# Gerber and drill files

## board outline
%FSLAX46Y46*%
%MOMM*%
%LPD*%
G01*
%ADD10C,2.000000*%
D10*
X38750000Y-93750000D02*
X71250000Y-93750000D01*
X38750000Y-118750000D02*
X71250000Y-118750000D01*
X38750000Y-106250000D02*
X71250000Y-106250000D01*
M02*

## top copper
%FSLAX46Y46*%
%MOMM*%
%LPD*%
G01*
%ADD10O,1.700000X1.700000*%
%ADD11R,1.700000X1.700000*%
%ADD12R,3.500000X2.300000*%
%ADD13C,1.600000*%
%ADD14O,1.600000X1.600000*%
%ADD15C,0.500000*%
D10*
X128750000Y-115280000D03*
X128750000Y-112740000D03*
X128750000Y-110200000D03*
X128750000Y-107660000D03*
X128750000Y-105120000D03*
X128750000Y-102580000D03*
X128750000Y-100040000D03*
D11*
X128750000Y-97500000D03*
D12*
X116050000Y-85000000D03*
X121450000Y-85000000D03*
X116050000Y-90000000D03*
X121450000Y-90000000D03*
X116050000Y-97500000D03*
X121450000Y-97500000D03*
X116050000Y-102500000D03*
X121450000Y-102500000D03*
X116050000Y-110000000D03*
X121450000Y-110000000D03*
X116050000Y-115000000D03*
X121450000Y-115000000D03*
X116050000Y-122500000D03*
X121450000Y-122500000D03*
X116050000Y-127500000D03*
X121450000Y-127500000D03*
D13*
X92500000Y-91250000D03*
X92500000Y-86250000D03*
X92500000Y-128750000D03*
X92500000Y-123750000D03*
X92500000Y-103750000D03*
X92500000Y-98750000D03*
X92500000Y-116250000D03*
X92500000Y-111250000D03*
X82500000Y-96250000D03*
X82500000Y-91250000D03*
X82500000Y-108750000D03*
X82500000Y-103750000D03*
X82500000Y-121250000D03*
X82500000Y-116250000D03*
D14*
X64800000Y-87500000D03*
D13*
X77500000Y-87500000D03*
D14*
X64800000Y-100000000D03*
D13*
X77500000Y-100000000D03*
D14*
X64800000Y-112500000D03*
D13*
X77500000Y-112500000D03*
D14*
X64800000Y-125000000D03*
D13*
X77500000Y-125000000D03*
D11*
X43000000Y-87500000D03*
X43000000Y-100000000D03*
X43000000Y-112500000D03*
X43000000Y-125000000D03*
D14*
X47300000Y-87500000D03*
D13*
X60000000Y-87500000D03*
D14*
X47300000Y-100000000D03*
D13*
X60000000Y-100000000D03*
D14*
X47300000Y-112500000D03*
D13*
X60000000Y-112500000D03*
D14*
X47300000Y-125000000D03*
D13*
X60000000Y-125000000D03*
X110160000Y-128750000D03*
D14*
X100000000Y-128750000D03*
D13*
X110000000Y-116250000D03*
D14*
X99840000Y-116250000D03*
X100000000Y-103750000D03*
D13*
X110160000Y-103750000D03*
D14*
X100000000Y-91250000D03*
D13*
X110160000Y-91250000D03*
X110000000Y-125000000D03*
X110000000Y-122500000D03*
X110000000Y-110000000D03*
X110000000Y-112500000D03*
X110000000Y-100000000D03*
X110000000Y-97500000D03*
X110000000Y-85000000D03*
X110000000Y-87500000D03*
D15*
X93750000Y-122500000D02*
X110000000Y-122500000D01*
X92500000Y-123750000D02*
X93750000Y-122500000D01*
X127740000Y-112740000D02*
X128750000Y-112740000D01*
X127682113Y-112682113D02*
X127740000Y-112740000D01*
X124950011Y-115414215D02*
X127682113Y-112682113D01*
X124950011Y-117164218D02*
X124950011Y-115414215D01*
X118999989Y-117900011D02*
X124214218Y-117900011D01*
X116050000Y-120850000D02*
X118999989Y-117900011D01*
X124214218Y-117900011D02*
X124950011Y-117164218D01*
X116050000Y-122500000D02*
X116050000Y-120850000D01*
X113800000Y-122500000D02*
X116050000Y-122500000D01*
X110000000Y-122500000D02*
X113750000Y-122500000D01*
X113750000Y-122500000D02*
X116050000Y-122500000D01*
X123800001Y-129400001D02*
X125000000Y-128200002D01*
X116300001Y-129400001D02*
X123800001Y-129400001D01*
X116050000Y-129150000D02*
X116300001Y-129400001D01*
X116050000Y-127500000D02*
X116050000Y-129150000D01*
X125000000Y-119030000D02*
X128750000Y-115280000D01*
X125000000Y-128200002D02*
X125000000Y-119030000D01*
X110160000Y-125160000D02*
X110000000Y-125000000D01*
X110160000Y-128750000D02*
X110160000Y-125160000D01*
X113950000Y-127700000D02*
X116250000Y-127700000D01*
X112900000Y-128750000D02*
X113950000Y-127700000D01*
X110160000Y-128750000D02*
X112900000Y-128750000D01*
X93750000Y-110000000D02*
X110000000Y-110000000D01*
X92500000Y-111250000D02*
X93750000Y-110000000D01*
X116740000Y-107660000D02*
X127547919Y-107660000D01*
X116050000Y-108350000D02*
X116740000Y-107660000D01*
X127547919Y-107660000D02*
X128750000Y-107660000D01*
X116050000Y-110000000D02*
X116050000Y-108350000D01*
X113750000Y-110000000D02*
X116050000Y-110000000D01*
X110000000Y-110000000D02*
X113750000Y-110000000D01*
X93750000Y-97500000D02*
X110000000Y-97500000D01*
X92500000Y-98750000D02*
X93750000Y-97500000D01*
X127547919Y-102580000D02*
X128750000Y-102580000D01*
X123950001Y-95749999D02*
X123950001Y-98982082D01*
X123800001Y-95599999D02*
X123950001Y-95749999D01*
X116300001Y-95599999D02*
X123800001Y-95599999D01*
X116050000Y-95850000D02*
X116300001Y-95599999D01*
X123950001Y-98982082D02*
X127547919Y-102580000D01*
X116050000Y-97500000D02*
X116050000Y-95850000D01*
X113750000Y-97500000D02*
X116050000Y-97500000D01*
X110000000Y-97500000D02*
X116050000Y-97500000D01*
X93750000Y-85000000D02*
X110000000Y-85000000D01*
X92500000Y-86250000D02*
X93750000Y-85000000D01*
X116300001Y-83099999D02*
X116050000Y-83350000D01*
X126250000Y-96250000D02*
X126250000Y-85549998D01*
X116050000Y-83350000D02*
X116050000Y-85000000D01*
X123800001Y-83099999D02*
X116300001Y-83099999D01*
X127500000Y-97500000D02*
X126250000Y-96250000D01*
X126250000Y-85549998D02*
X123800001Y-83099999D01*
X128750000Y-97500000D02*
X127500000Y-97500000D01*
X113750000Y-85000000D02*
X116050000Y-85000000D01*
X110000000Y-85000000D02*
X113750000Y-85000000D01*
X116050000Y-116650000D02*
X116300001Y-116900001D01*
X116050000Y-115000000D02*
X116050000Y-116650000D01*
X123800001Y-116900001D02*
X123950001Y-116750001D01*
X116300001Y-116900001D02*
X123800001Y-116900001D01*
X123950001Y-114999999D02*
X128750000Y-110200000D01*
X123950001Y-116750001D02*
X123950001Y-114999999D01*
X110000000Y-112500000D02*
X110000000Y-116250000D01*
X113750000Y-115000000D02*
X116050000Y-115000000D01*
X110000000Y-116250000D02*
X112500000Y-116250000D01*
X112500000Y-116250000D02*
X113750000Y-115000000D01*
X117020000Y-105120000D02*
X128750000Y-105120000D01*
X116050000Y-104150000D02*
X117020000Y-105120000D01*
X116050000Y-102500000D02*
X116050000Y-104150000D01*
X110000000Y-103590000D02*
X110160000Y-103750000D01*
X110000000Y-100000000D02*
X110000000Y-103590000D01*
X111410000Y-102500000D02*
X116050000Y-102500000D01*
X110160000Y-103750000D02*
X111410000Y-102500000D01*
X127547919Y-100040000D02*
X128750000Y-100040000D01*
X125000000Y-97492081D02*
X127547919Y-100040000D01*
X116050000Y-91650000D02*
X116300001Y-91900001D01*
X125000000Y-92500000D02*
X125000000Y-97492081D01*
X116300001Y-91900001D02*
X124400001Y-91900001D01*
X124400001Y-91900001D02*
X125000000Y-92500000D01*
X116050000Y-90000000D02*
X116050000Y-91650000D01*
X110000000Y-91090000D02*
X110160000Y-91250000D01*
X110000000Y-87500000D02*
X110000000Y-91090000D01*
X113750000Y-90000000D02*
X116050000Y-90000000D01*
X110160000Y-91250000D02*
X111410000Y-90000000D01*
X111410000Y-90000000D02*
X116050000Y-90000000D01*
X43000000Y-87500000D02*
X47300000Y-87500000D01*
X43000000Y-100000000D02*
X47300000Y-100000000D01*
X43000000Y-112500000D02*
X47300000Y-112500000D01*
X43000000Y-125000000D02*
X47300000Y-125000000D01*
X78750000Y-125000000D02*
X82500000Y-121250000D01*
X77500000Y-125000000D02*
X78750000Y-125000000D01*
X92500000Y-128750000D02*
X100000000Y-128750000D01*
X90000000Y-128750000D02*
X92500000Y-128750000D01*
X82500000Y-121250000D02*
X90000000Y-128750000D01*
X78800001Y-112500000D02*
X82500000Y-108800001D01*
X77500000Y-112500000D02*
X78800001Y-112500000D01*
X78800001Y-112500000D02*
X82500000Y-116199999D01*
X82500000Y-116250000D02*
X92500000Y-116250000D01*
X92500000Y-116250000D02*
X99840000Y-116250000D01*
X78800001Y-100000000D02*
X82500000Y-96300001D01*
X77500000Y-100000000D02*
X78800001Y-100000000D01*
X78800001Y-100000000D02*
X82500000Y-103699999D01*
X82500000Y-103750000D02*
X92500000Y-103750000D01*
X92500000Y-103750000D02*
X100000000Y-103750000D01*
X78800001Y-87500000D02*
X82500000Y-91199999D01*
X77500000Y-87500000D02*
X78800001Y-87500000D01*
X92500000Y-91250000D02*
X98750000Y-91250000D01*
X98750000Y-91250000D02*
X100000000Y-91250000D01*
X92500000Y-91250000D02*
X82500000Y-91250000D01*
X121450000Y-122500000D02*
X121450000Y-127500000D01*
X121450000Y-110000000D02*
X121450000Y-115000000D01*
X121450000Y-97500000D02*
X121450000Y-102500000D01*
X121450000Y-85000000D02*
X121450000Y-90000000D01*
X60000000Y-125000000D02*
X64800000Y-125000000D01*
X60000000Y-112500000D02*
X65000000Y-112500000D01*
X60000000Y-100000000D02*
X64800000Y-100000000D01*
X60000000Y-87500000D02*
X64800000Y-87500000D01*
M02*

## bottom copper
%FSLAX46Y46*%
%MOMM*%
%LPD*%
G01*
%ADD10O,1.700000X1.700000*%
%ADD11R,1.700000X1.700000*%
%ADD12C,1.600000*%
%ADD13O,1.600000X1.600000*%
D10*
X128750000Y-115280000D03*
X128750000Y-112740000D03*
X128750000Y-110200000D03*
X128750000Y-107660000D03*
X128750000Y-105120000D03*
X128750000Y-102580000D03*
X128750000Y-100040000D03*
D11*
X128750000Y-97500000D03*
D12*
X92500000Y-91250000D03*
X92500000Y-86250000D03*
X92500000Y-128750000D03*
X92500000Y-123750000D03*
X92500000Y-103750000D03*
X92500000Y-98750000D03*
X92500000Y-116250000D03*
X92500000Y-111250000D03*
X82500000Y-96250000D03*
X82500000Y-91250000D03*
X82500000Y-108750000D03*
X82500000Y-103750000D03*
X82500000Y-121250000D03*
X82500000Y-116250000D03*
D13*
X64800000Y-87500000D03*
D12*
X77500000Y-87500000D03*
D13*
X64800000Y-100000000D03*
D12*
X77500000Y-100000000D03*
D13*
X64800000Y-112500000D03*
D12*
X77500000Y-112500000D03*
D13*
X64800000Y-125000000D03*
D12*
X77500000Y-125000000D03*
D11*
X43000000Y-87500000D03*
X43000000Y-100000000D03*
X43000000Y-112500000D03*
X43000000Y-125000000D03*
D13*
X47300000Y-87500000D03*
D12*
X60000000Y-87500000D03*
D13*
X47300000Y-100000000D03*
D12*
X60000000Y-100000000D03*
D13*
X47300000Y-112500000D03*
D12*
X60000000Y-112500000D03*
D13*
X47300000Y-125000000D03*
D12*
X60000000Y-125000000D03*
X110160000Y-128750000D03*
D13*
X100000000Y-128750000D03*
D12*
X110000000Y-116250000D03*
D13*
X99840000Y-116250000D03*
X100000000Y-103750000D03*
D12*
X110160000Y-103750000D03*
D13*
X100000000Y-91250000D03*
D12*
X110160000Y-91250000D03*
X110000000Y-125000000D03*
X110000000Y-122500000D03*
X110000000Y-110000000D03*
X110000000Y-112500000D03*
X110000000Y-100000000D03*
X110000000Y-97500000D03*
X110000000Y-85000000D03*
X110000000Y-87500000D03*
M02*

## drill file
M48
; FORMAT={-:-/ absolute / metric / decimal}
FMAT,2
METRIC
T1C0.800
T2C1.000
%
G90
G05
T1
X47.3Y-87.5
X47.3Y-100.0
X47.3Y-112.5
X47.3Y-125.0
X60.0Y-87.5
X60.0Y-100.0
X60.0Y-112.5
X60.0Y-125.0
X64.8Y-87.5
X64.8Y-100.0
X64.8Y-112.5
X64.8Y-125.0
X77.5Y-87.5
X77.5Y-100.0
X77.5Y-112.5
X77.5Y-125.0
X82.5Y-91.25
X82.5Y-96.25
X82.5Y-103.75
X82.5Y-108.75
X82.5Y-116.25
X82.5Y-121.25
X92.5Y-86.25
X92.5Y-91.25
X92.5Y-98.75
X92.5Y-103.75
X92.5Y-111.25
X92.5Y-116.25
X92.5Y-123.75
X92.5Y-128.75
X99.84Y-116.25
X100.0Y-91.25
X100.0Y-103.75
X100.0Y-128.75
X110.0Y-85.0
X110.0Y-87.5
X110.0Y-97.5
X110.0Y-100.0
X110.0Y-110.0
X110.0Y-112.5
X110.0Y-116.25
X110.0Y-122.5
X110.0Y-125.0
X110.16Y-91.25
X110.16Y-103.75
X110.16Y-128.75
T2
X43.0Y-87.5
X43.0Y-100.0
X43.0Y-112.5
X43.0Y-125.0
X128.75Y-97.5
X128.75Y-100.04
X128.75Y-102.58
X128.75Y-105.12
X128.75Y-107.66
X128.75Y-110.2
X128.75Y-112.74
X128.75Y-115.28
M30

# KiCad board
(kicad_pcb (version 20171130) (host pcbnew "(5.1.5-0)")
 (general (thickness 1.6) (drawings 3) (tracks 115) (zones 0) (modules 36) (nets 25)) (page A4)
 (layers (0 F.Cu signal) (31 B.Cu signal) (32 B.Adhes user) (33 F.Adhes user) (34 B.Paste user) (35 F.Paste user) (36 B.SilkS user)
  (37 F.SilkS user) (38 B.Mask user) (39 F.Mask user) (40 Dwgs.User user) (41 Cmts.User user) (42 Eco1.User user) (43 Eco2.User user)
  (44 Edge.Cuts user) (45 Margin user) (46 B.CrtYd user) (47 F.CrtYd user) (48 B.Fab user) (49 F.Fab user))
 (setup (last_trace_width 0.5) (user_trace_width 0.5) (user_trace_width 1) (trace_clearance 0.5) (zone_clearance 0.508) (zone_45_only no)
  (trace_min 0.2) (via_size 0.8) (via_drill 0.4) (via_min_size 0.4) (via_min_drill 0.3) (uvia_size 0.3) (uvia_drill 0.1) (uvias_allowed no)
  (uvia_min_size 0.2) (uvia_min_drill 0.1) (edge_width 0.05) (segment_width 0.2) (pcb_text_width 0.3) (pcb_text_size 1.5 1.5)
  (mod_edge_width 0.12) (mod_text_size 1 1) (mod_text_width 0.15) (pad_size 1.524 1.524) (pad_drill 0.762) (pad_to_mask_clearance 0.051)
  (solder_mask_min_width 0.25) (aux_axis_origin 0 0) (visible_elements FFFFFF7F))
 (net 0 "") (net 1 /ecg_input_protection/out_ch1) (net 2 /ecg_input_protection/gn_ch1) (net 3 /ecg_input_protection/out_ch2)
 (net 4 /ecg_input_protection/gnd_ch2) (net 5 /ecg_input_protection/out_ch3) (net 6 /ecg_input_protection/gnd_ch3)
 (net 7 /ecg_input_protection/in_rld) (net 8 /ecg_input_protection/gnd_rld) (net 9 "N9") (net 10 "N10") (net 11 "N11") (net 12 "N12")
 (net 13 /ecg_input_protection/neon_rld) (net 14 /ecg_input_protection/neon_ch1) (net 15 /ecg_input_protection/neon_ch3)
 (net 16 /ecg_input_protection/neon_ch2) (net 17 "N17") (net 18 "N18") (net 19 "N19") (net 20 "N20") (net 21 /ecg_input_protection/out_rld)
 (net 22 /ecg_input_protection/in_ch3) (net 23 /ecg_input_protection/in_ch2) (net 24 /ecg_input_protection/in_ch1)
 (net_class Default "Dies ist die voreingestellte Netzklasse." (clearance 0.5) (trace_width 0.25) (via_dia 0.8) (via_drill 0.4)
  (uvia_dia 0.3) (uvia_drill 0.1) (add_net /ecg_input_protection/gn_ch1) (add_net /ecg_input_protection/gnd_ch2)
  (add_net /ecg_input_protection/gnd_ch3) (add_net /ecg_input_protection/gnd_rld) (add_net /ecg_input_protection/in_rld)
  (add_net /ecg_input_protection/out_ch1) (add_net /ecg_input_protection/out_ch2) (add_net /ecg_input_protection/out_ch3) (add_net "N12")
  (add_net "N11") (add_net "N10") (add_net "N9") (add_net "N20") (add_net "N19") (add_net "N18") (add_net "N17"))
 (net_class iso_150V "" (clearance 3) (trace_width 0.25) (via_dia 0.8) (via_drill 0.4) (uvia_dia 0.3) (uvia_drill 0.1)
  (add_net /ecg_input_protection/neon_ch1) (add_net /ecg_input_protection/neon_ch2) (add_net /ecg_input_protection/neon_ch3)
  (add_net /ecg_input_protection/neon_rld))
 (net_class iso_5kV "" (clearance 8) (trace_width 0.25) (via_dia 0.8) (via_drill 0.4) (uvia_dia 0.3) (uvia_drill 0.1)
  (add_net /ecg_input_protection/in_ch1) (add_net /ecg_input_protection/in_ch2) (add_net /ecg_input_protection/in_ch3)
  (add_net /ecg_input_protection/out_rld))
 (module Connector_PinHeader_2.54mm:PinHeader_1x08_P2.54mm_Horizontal (layer F.Cu) (at 128.75 97.5)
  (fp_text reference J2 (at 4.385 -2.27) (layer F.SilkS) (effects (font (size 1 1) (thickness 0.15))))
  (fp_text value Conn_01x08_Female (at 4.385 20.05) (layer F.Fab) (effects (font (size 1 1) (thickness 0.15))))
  (pad 8 thru_hole oval (at 0 17.78) (size 1.7 1.7) (drill 1) (layers *.Cu *.Mask) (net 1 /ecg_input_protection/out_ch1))
  (pad 7 thru_hole oval (at 0 15.24) (size 1.7 1.7) (drill 1) (layers *.Cu *.Mask) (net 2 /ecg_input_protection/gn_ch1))
  (pad 6 thru_hole oval (at 0 12.7) (size 1.7 1.7) (drill 1) (layers *.Cu *.Mask) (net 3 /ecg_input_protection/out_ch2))
  (pad 5 thru_hole oval (at 0 10.16) (size 1.7 1.7) (drill 1) (layers *.Cu *.Mask) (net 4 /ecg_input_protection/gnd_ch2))
  (pad 4 thru_hole oval (at 0 7.62) (size 1.7 1.7) (drill 1) (layers *.Cu *.Mask) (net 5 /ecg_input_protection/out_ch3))
  (pad 3 thru_hole oval (at 0 5.08) (size 1.7 1.7) (drill 1) (layers *.Cu *.Mask) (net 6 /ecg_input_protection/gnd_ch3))
  (pad 2 thru_hole oval (at 0 2.54) (size 1.7 1.7) (drill 1) (layers *.Cu *.Mask) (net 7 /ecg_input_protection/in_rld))
  (pad 1 thru_hole rect (at 0 0) (size 1.7 1.7) (drill 1) (layers *.Cu *.Mask) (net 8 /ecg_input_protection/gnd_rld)))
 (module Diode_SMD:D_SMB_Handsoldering (layer F.Cu) (at 118.75 85 180)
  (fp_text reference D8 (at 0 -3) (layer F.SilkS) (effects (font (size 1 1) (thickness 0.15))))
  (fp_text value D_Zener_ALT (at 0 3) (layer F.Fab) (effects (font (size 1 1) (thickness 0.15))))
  (pad 2 smd rect (at 2.7 0 180) (size 3.5 2.3) (layers F.Cu F.Paste F.Mask) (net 8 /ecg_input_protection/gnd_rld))
  (pad 1 smd rect (at -2.7 0 180) (size 3.5 2.3) (layers F.Cu F.Paste F.Mask) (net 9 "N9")))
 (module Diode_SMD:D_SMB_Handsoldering (layer F.Cu) (at 118.75 90 180)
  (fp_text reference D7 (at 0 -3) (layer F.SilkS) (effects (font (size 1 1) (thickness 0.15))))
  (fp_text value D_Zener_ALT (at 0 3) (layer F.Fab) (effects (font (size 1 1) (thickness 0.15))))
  (pad 2 smd rect (at 2.7 0 180) (size 3.5 2.3) (layers F.Cu F.Paste F.Mask) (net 7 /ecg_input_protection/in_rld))
  (pad 1 smd rect (at -2.7 0 180) (size 3.5 2.3) (layers F.Cu F.Paste F.Mask) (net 9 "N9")))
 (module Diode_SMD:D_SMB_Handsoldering (layer F.Cu) (at 118.75 97.5 180)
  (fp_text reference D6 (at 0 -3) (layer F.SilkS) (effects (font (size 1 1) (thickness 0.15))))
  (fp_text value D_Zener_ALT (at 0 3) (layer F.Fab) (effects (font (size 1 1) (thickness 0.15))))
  (pad 2 smd rect (at 2.7 0 180) (size 3.5 2.3) (layers F.Cu F.Paste F.Mask) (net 6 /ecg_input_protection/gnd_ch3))
  (pad 1 smd rect (at -2.7 0 180) (size 3.5 2.3) (layers F.Cu F.Paste F.Mask) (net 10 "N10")))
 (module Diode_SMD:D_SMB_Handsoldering (layer F.Cu) (at 118.75 102.5 180)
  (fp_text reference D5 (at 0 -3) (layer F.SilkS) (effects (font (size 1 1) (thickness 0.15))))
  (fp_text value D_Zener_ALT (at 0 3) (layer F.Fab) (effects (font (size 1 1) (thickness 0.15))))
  (pad 2 smd rect (at 2.7 0 180) (size 3.5 2.3) (layers F.Cu F.Paste F.Mask) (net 5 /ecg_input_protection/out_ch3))
  (pad 1 smd rect (at -2.7 0 180) (size 3.5 2.3) (layers F.Cu F.Paste F.Mask) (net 10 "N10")))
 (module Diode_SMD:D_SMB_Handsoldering (layer F.Cu) (at 118.75 110 180)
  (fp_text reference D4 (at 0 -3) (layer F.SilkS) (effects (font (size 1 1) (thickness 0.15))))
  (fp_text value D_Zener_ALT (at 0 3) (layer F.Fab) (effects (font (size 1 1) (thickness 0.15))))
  (pad 2 smd rect (at 2.7 0 180) (size 3.5 2.3) (layers F.Cu F.Paste F.Mask) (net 4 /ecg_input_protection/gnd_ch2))
  (pad 1 smd rect (at -2.7 0 180) (size 3.5 2.3) (layers F.Cu F.Paste F.Mask) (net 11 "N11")))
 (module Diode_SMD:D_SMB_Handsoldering (layer F.Cu) (at 118.75 115 180)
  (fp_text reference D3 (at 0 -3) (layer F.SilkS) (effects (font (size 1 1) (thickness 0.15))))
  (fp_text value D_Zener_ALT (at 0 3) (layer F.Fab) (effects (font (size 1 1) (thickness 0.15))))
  (pad 2 smd rect (at 2.7 0 180) (size 3.5 2.3) (layers F.Cu F.Paste F.Mask) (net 3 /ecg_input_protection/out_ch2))
  (pad 1 smd rect (at -2.7 0 180) (size 3.5 2.3) (layers F.Cu F.Paste F.Mask) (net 11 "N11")))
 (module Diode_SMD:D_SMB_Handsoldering (layer F.Cu) (at 118.75 122.5 180)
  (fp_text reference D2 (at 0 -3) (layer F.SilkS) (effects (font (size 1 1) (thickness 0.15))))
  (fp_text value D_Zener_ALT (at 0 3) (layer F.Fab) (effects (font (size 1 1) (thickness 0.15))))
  (pad 2 smd rect (at 2.7 0 180) (size 3.5 2.3) (layers F.Cu F.Paste F.Mask) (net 2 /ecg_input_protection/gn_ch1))
  (pad 1 smd rect (at -2.7 0 180) (size 3.5 2.3) (layers F.Cu F.Paste F.Mask) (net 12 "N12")))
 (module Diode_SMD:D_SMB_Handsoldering (layer F.Cu) (at 118.75 127.5 180)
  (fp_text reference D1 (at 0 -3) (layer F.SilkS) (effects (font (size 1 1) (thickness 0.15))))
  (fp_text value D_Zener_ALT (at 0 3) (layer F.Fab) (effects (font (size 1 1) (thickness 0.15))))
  (pad 2 smd rect (at 2.7 0 180) (size 3.5 2.3) (layers F.Cu F.Paste F.Mask) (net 1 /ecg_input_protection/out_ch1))
  (pad 1 smd rect (at -2.7 0 180) (size 3.5 2.3) (layers F.Cu F.Paste F.Mask) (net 12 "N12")))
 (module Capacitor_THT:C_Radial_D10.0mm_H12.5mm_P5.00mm (layer F.Cu) (at 92.5 86.25 270)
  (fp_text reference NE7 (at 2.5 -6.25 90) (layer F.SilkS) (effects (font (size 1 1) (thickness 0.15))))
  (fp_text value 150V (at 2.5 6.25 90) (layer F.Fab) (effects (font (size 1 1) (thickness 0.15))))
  (pad 2 thru_hole circle (at 5 0 270) (size 1.6 1.6) (drill 0.8) (layers *.Cu *.Mask) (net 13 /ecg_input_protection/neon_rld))
  (pad 1 thru_hole circle (at 0 0 270) (size 1.6 1.6) (drill 0.8) (layers *.Cu *.Mask) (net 8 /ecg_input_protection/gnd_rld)))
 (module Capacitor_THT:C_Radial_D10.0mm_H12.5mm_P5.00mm (layer F.Cu) (at 92.5 123.75 270)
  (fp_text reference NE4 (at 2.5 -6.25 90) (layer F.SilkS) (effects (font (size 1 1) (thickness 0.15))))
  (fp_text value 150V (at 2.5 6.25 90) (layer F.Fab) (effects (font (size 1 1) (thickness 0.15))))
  (pad 2 thru_hole circle (at 5 0 270) (size 1.6 1.6) (drill 0.8) (layers *.Cu *.Mask) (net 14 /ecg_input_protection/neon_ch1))
  (pad 1 thru_hole circle (at 0 0 270) (size 1.6 1.6) (drill 0.8) (layers *.Cu *.Mask) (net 2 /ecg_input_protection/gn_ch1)))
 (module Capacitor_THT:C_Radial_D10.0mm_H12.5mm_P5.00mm (layer F.Cu) (at 92.5 98.75 270)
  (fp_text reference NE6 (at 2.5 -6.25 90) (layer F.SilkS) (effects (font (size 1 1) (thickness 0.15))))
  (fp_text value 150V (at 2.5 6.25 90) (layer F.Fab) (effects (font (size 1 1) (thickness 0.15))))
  (pad 2 thru_hole circle (at 5 0 270) (size 1.6 1.6) (drill 0.8) (layers *.Cu *.Mask) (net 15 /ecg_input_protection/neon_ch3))
  (pad 1 thru_hole circle (at 0 0 270) (size 1.6 1.6) (drill 0.8) (layers *.Cu *.Mask) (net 6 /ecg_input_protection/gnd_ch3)))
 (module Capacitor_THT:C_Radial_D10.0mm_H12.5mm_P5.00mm (layer F.Cu) (at 92.5 111.25 270)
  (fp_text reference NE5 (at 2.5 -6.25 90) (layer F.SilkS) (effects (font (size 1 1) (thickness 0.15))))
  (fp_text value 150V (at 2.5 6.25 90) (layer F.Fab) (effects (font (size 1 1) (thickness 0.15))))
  (pad 2 thru_hole circle (at 5 0 270) (size 1.6 1.6) (drill 0.8) (layers *.Cu *.Mask) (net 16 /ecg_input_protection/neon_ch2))
  (pad 1 thru_hole circle (at 0 0 270) (size 1.6 1.6) (drill 0.8) (layers *.Cu *.Mask) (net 4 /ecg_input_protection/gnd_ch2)))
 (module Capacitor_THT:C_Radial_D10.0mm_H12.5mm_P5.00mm (layer F.Cu) (at 82.5 91.25 270)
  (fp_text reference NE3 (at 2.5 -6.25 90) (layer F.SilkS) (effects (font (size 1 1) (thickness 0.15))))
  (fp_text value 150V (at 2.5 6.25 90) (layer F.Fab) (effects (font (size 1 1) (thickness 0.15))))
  (pad 2 thru_hole circle (at 5 0 270) (size 1.6 1.6) (drill 0.8) (layers *.Cu *.Mask) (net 15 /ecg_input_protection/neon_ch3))
  (pad 1 thru_hole circle (at 0 0 270) (size 1.6 1.6) (drill 0.8) (layers *.Cu *.Mask) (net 13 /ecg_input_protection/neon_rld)))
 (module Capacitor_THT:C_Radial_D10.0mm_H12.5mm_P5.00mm (layer F.Cu) (at 82.5 103.75 270)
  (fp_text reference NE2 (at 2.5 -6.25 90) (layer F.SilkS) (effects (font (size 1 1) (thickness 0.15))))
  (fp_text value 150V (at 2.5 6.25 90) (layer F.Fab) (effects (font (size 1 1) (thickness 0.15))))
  (pad 2 thru_hole circle (at 5 0 270) (size 1.6 1.6) (drill 0.8) (layers *.Cu *.Mask) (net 16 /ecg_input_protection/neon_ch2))
  (pad 1 thru_hole circle (at 0 0 270) (size 1.6 1.6) (drill 0.8) (layers *.Cu *.Mask) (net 15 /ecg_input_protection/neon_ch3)))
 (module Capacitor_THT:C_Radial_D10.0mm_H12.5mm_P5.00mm (layer F.Cu) (at 82.5 116.25 270)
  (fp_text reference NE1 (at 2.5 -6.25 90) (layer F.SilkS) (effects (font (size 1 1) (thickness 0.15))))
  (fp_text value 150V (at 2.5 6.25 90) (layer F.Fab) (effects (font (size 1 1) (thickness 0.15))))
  (pad 2 thru_hole circle (at 5 0 270) (size 1.6 1.6) (drill 0.8) (layers *.Cu *.Mask) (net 14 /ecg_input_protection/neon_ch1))
  (pad 1 thru_hole circle (at 0 0 270) (size 1.6 1.6) (drill 0.8) (layers *.Cu *.Mask) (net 16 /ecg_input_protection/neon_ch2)))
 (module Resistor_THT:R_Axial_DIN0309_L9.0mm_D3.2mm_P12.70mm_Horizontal (layer F.Cu) (at 77.5 87.5 180)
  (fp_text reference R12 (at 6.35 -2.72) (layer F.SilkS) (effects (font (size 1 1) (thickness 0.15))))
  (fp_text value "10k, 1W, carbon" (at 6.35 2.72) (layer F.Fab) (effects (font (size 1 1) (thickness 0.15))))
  (pad 2 thru_hole oval (at 12.7 0 180) (size 1.6 1.6) (drill 0.8) (layers *.Cu *.Mask) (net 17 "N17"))
  (pad 1 thru_hole circle (at 0 0 180) (size 1.6 1.6) (drill 0.8) (layers *.Cu *.Mask) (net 13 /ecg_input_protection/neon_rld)))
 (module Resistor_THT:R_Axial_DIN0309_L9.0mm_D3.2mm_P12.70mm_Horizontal (layer F.Cu) (at 77.5 100 180)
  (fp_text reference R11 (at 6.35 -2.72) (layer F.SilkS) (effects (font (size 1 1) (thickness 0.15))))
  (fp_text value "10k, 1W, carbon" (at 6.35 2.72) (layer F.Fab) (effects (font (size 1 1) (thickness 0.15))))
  (pad 2 thru_hole oval (at 12.7 0 180) (size 1.6 1.6) (drill 0.8) (layers *.Cu *.Mask) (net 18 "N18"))
  (pad 1 thru_hole circle (at 0 0 180) (size 1.6 1.6) (drill 0.8) (layers *.Cu *.Mask) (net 15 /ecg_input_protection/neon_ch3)))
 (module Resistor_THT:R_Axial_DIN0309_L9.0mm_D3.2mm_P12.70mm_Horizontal (layer F.Cu) (at 77.5 112.5 180)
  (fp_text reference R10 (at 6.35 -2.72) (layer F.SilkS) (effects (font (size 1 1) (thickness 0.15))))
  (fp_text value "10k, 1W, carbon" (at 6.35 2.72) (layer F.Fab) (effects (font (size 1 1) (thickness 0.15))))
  (pad 2 thru_hole oval (at 12.7 0 180) (size 1.6 1.6) (drill 0.8) (layers *.Cu *.Mask) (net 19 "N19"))
  (pad 1 thru_hole circle (at 0 0 180) (size 1.6 1.6) (drill 0.8) (layers *.Cu *.Mask) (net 16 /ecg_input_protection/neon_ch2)))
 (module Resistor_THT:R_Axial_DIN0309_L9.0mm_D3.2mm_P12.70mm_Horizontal (layer F.Cu) (at 77.5 125 180)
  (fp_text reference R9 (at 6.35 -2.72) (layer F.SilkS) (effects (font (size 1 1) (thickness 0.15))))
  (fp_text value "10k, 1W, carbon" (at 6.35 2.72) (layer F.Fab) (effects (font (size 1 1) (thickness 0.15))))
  (pad 2 thru_hole oval (at 12.7 0 180) (size 1.6 1.6) (drill 0.8) (layers *.Cu *.Mask) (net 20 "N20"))
  (pad 1 thru_hole circle (at 0 0 180) (size 1.6 1.6) (drill 0.8) (layers *.Cu *.Mask) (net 14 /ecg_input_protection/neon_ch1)))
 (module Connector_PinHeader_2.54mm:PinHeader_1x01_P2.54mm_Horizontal (layer F.Cu) (at 43 87.5 180)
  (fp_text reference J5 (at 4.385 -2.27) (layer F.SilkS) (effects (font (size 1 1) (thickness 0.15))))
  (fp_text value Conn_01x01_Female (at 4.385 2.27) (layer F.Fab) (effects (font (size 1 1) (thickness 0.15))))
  (pad 1 thru_hole rect (at 0 0 180) (size 1.7 1.7) (drill 1) (layers *.Cu *.Mask) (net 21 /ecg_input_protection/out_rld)))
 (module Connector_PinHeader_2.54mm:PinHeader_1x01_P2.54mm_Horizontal (layer F.Cu) (at 43 100 180)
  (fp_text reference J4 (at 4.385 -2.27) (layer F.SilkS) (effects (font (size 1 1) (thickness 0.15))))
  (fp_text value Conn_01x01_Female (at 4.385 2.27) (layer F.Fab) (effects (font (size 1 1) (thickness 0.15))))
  (pad 1 thru_hole rect (at 0 0 180) (size 1.7 1.7) (drill 1) (layers *.Cu *.Mask) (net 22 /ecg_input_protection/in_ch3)))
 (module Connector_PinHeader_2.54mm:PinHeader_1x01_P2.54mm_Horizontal (layer F.Cu) (at 43 112.5 180)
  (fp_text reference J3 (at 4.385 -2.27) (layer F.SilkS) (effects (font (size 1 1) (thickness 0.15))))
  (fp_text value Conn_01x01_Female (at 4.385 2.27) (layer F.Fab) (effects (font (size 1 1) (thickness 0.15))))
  (pad 1 thru_hole rect (at 0 0 180) (size 1.7 1.7) (drill 1) (layers *.Cu *.Mask) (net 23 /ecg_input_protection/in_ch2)))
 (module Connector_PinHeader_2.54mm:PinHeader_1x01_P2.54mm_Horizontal (layer F.Cu) (at 43 125 180)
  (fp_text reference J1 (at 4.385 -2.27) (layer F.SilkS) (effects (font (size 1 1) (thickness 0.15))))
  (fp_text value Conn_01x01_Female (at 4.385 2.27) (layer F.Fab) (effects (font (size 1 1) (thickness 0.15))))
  (pad 1 thru_hole rect (at 0 0 180) (size 1.7 1.7) (drill 1) (layers *.Cu *.Mask) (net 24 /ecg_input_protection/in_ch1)))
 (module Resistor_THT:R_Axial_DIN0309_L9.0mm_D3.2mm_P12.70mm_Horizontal (layer F.Cu) (at 60 87.5 180)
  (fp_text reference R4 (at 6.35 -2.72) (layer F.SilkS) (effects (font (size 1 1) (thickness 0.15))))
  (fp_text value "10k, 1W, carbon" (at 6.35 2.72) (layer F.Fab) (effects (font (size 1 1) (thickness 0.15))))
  (pad 2 thru_hole oval (at 12.7 0 180) (size 1.6 1.6) (drill 0.8) (layers *.Cu *.Mask) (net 21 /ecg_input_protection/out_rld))
  (pad 1 thru_hole circle (at 0 0 180) (size 1.6 1.6) (drill 0.8) (layers *.Cu *.Mask) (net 17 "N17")))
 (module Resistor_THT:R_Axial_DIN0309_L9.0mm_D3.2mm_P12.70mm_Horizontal (layer F.Cu) (at 60 100 180)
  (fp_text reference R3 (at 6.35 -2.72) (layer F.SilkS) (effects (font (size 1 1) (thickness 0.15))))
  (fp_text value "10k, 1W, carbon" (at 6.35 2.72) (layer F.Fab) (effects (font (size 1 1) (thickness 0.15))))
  (pad 2 thru_hole oval (at 12.7 0 180) (size 1.6 1.6) (drill 0.8) (layers *.Cu *.Mask) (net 22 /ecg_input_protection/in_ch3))
  (pad 1 thru_hole circle (at 0 0 180) (size 1.6 1.6) (drill 0.8) (layers *.Cu *.Mask) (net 18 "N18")))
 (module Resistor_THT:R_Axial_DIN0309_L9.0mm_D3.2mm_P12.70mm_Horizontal (layer F.Cu) (at 60 112.5 180)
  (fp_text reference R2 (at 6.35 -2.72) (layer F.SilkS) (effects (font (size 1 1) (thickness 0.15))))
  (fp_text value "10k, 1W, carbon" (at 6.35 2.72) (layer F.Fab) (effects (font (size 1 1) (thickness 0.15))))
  (pad 2 thru_hole oval (at 12.7 0 180) (size 1.6 1.6) (drill 0.8) (layers *.Cu *.Mask) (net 23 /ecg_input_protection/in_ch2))
  (pad 1 thru_hole circle (at 0 0 180) (size 1.6 1.6) (drill 0.8) (layers *.Cu *.Mask) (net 19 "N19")))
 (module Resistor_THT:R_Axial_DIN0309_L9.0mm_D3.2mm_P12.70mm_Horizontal (layer F.Cu) (at 60 125 180)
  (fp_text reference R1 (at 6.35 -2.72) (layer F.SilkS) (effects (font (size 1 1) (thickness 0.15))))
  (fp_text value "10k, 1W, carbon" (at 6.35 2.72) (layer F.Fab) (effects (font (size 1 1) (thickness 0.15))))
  (pad 2 thru_hole oval (at 12.7 0 180) (size 1.6 1.6) (drill 0.8) (layers *.Cu *.Mask) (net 24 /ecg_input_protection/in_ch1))
  (pad 1 thru_hole circle (at 0 0 180) (size 1.6 1.6) (drill 0.8) (layers *.Cu *.Mask) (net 20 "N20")))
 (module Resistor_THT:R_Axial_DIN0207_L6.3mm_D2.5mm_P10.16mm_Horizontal (layer F.Cu) (at 110.16 128.75 180)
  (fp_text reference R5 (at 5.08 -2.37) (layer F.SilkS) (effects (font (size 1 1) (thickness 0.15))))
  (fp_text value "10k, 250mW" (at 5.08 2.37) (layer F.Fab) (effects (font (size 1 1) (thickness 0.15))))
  (pad 1 thru_hole circle (at 0 0 180) (size 1.6 1.6) (drill 0.8) (layers *.Cu *.Mask) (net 1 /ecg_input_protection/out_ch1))
  (pad 2 thru_hole oval (at 10.16 0 180) (size 1.6 1.6) (drill 0.8) (layers *.Cu *.Mask) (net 14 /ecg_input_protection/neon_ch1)))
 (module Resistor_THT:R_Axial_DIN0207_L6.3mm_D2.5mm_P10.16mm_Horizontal (layer F.Cu) (at 110 116.25 180)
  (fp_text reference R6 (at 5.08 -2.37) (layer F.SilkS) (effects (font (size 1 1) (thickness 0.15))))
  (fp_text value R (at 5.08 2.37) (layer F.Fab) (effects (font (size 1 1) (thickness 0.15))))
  (pad 1 thru_hole circle (at 0 0 180) (size 1.6 1.6) (drill 0.8) (layers *.Cu *.Mask) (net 3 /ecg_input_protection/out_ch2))
  (pad 2 thru_hole oval (at 10.16 0 180) (size 1.6 1.6) (drill 0.8) (layers *.Cu *.Mask) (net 16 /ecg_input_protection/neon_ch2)))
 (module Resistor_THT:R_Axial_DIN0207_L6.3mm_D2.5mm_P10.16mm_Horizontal (layer F.Cu) (at 110.16 103.75 180)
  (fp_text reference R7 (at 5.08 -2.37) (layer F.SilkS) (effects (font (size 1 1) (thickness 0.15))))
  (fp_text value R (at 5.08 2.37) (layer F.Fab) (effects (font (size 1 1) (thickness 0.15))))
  (pad 2 thru_hole oval (at 10.16 0 180) (size 1.6 1.6) (drill 0.8) (layers *.Cu *.Mask) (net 15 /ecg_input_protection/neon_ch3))
  (pad 1 thru_hole circle (at 0 0 180) (size 1.6 1.6) (drill 0.8) (layers *.Cu *.Mask) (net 5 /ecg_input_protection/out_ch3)))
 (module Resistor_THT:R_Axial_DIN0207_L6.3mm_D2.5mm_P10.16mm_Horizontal (layer F.Cu) (at 110.16 91.25 180)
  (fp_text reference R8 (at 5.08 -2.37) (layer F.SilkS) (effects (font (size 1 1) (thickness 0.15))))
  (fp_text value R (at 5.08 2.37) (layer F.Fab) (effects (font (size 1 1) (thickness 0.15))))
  (pad 2 thru_hole oval (at 10.16 0 180) (size 1.6 1.6) (drill 0.8) (layers *.Cu *.Mask) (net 13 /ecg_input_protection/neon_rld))
  (pad 1 thru_hole circle (at 0 0 180) (size 1.6 1.6) (drill 0.8) (layers *.Cu *.Mask) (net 7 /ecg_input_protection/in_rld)))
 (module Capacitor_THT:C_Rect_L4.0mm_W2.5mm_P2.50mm (layer F.Cu) (at 110 125 90)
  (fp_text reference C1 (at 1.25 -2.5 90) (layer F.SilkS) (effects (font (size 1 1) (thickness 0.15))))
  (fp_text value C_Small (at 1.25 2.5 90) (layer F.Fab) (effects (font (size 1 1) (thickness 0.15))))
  (pad 1 thru_hole circle (at 0 0 90) (size 1.6 1.6) (drill 0.8) (layers *.Cu *.Mask) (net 1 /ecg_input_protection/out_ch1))
  (pad 2 thru_hole circle (at 2.5 0 90) (size 1.6 1.6) (drill 0.8) (layers *.Cu *.Mask) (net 2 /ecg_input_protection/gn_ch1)))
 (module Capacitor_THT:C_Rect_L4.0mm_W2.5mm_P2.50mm (layer F.Cu) (at 110 112.5 90)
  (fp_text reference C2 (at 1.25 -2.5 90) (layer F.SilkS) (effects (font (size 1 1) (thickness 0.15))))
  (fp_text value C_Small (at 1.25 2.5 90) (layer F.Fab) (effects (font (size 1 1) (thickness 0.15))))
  (pad 2 thru_hole circle (at 2.5 0 90) (size 1.6 1.6) (drill 0.8) (layers *.Cu *.Mask) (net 4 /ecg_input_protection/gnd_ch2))
  (pad 1 thru_hole circle (at 0 0 90) (size 1.6 1.6) (drill 0.8) (layers *.Cu *.Mask) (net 3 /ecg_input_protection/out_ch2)))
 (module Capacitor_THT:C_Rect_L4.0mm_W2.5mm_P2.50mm (layer F.Cu) (at 110 100 90)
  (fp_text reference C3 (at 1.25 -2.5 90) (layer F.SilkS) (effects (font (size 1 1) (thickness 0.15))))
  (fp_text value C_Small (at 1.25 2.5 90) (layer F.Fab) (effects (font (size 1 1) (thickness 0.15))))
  (pad 1 thru_hole circle (at 0 0 90) (size 1.6 1.6) (drill 0.8) (layers *.Cu *.Mask) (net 5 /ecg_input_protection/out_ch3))
  (pad 2 thru_hole circle (at 2.5 0 90) (size 1.6 1.6) (drill 0.8) (layers *.Cu *.Mask) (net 6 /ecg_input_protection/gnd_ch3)))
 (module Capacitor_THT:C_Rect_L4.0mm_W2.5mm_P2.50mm (layer F.Cu) (at 110 87.5 90)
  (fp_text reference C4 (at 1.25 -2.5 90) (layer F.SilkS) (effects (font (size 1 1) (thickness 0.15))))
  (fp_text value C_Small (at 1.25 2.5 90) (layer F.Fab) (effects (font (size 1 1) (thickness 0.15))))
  (pad 2 thru_hole circle (at 2.5 0 90) (size 1.6 1.6) (drill 0.8) (layers *.Cu *.Mask) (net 8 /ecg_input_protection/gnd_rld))
  (pad 1 thru_hole circle (at 0 0 90) (size 1.6 1.6) (drill 0.8) (layers *.Cu *.Mask) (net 7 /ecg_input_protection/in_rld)))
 (gr_line (start 38.75 93.75) (end 71.25 93.75) (layer Edge.Cuts) (width 2))
 (gr_line (start 38.75 118.75) (end 71.25 118.75) (layer Edge.Cuts) (width 2))
 (gr_line (start 38.75 106.25) (end 71.25 106.25) (layer Edge.Cuts) (width 2))
 (segment (start 93.75 122.5) (end 110 122.5) (width 0.5) (layer F.Cu) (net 2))
 (segment (start 92.5 123.75) (end 93.75 122.5) (width 0.5) (layer F.Cu) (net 2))
 (segment (start 127.74 112.74) (end 128.75 112.74) (width 0.5) (layer F.Cu) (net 2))
 (segment (start 127.682113 112.682113) (end 127.74 112.74) (width 0.5) (layer F.Cu) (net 2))
 (segment (start 124.950011 115.414215) (end 127.682113 112.682113) (width 0.5) (layer F.Cu) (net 2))
 (segment (start 124.950011 117.164218) (end 124.950011 115.414215) (width 0.5) (layer F.Cu) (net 2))
 (segment (start 118.999989 117.900011) (end 124.214218 117.900011) (width 0.5) (layer F.Cu) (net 2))
 (segment (start 116.05 120.85) (end 118.999989 117.900011) (width 0.5) (layer F.Cu) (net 2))
 (segment (start 124.214218 117.900011) (end 124.950011 117.164218) (width 0.5) (layer F.Cu) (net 2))
 (segment (start 116.05 122.5) (end 116.05 120.85) (width 0.5) (layer F.Cu) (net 2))
 (segment (start 113.8 122.5) (end 116.05 122.5) (width 0.5) (layer F.Cu) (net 2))
 (segment (start 110 122.5) (end 113.75 122.5) (width 0.5) (layer F.Cu) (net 2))
 (segment (start 113.75 122.5) (end 116.05 122.5) (width 0.5) (layer F.Cu) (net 2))
 (segment (start 123.800001 129.400001) (end 125 128.200002) (width 0.5) (layer F.Cu) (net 1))
 (segment (start 116.300001 129.400001) (end 123.800001 129.400001) (width 0.5) (layer F.Cu) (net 1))
 (segment (start 116.05 129.15) (end 116.300001 129.400001) (width 0.5) (layer F.Cu) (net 1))
 (segment (start 116.05 127.5) (end 116.05 129.15) (width 0.5) (layer F.Cu) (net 1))
 (segment (start 125 119.03) (end 128.75 115.28) (width 0.5) (layer F.Cu) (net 1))
 (segment (start 125 128.200002) (end 125 119.03) (width 0.5) (layer F.Cu) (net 1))
 (segment (start 110.16 125.16) (end 110 125) (width 0.5) (layer F.Cu) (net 1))
 (segment (start 110.16 128.75) (end 110.16 125.16) (width 0.5) (layer F.Cu) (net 1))
 (segment (start 113.95 127.7) (end 116.25 127.7) (width 0.5) (layer F.Cu) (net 1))
 (segment (start 112.9 128.75) (end 113.95 127.7) (width 0.5) (layer F.Cu) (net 1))
 (segment (start 110.16 128.75) (end 112.9 128.75) (width 0.5) (layer F.Cu) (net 1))
 (segment (start 93.75 110) (end 110 110) (width 0.5) (layer F.Cu) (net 4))
 (segment (start 92.5 111.25) (end 93.75 110) (width 0.5) (layer F.Cu) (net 4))
 (segment (start 116.74 107.66) (end 127.547919 107.66) (width 0.5) (layer F.Cu) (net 4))
 (segment (start 116.05 108.35) (end 116.74 107.66) (width 0.5) (layer F.Cu) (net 4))
 (segment (start 127.547919 107.66) (end 128.75 107.66) (width 0.5) (layer F.Cu) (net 4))
 (segment (start 116.05 110) (end 116.05 108.35) (width 0.5) (layer F.Cu) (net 4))
 (segment (start 113.75 110) (end 116.05 110) (width 0.5) (layer F.Cu) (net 4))
 (segment (start 110 110) (end 113.75 110) (width 0.5) (layer F.Cu) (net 4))
 (segment (start 93.75 97.5) (end 110 97.5) (width 0.5) (layer F.Cu) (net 6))
 (segment (start 92.5 98.75) (end 93.75 97.5) (width 0.5) (layer F.Cu) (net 6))
 (segment (start 127.547919 102.58) (end 128.75 102.58) (width 0.5) (layer F.Cu) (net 6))
 (segment (start 123.950001 95.749999) (end 123.950001 98.982082) (width 0.5) (layer F.Cu) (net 6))
 (segment (start 123.800001 95.599999) (end 123.950001 95.749999) (width 0.5) (layer F.Cu) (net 6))
 (segment (start 116.300001 95.599999) (end 123.800001 95.599999) (width 0.5) (layer F.Cu) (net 6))
 (segment (start 116.05 95.85) (end 116.300001 95.599999) (width 0.5) (layer F.Cu) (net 6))
 (segment (start 123.950001 98.982082) (end 127.547919 102.58) (width 0.5) (layer F.Cu) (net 6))
 (segment (start 116.05 97.5) (end 116.05 95.85) (width 0.5) (layer F.Cu) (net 6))
 (segment (start 113.75 97.5) (end 116.05 97.5) (width 0.5) (layer F.Cu) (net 6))
 (segment (start 110 97.5) (end 116.05 97.5) (width 0.5) (layer F.Cu) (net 6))
 (segment (start 93.75 85) (end 110 85) (width 0.5) (layer F.Cu) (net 8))
 (segment (start 92.5 86.25) (end 93.75 85) (width 0.5) (layer F.Cu) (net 8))
 (segment (start 116.300001 83.099999) (end 116.05 83.35) (width 0.5) (layer F.Cu) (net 8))
 (segment (start 126.25 96.25) (end 126.25 85.549998) (width 0.5) (layer F.Cu) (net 8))
 (segment (start 116.05 83.35) (end 116.05 85) (width 0.5) (layer F.Cu) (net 8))
 (segment (start 123.800001 83.099999) (end 116.300001 83.099999) (width 0.5) (layer F.Cu) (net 8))
 (segment (start 127.5 97.5) (end 126.25 96.25) (width 0.5) (layer F.Cu) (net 8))
 (segment (start 126.25 85.549998) (end 123.800001 83.099999) (width 0.5) (layer F.Cu) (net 8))
 (segment (start 128.75 97.5) (end 127.5 97.5) (width 0.5) (layer F.Cu) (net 8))
 (segment (start 113.75 85) (end 116.05 85) (width 0.5) (layer F.Cu) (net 8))
 (segment (start 110 85) (end 113.75 85) (width 0.5) (layer F.Cu) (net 8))
 (segment (start 116.05 116.65) (end 116.300001 116.900001) (width 0.5) (layer F.Cu) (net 3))
 (segment (start 116.05 115) (end 116.05 116.65) (width 0.5) (layer F.Cu) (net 3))
 (segment (start 123.800001 116.900001) (end 123.950001 116.750001) (width 0.5) (layer F.Cu) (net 3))
 (segment (start 116.300001 116.900001) (end 123.800001 116.900001) (width 0.5) (layer F.Cu) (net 3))
 (segment (start 123.950001 114.999999) (end 128.75 110.2) (width 0.5) (layer F.Cu) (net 3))
 (segment (start 123.950001 116.750001) (end 123.950001 114.999999) (width 0.5) (layer F.Cu) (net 3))
 (segment (start 110 112.5) (end 110 116.25) (width 0.5) (layer F.Cu) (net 3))
 (segment (start 113.75 115) (end 116.05 115) (width 0.5) (layer F.Cu) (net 3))
 (segment (start 110 116.25) (end 112.5 116.25) (width 0.5) (layer F.Cu) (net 3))
 (segment (start 112.5 116.25) (end 113.75 115) (width 0.5) (layer F.Cu) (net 3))
 (segment (start 117.02 105.12) (end 128.75 105.12) (width 0.5) (layer F.Cu) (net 5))
 (segment (start 116.05 104.15) (end 117.02 105.12) (width 0.5) (layer F.Cu) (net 5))
 (segment (start 116.05 102.5) (end 116.05 104.15) (width 0.5) (layer F.Cu) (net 5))
 (segment (start 110 103.59) (end 110.16 103.75) (width 0.5) (layer F.Cu) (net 5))
 (segment (start 110 100) (end 110 103.59) (width 0.5) (layer F.Cu) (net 5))
 (segment (start 111.41 102.5) (end 116.05 102.5) (width 0.5) (layer F.Cu) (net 5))
 (segment (start 110.16 103.75) (end 111.41 102.5) (width 0.5) (layer F.Cu) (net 5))
 (segment (start 127.547919 100.04) (end 128.75 100.04) (width 0.5) (layer F.Cu) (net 7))
 (segment (start 125 97.492081) (end 127.547919 100.04) (width 0.5) (layer F.Cu) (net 7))
 (segment (start 116.05 91.65) (end 116.300001 91.900001) (width 0.5) (layer F.Cu) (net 7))
 (segment (start 125 92.5) (end 125 97.492081) (width 0.5) (layer F.Cu) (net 7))
 (segment (start 116.300001 91.900001) (end 124.400001 91.900001) (width 0.5) (layer F.Cu) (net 7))
 (segment (start 124.400001 91.900001) (end 125 92.5) (width 0.5) (layer F.Cu) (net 7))
 (segment (start 116.05 90) (end 116.05 91.65) (width 0.5) (layer F.Cu) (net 7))
 (segment (start 110 91.09) (end 110.16 91.25) (width 0.5) (layer F.Cu) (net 7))
 (segment (start 110 87.5) (end 110 91.09) (width 0.5) (layer F.Cu) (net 7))
 (segment (start 113.75 90) (end 116.05 90) (width 0.5) (layer F.Cu) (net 7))
 (segment (start 110.16 91.25) (end 111.41 90) (width 0.5) (layer F.Cu) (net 7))
 (segment (start 111.41 90) (end 116.05 90) (width 0.5) (layer F.Cu) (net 7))
 (segment (start 43 87.5) (end 47.3 87.5) (width 0.5) (layer F.Cu) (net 21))
 (segment (start 43 100) (end 47.3 100) (width 0.5) (layer F.Cu) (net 22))
 (segment (start 43 112.5) (end 47.3 112.5) (width 0.5) (layer F.Cu) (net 23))
 (segment (start 43 125) (end 47.3 125) (width 0.5) (layer F.Cu) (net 24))
 (segment (start 78.75 125) (end 82.5 121.25) (width 0.5) (layer F.Cu) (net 14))
 (segment (start 77.5 125) (end 78.75 125) (width 0.5) (layer F.Cu) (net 14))
 (segment (start 92.5 128.75) (end 100 128.75) (width 0.5) (layer F.Cu) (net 14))
 (segment (start 90 128.75) (end 92.5 128.75) (width 0.5) (layer F.Cu) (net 14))
 (segment (start 82.5 121.25) (end 90 128.75) (width 0.5) (layer F.Cu) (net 14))
 (segment (start 78.800001 112.5) (end 82.5 108.800001) (width 0.5) (layer F.Cu) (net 16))
 (segment (start 77.5 112.5) (end 78.800001 112.5) (width 0.5) (layer F.Cu) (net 16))
 (segment (start 78.800001 112.5) (end 82.5 116.199999) (width 0.5) (layer F.Cu) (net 16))
 (segment (start 82.5 116.25) (end 92.5 116.25) (width 0.5) (layer F.Cu) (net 16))
 (segment (start 92.5 116.25) (end 99.84 116.25) (width 0.5) (layer F.Cu) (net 16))
 (segment (start 78.800001 100) (end 82.5 96.300001) (width 0.5) (layer F.Cu) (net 15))
 (segment (start 77.5 100) (end 78.800001 100) (width 0.5) (layer F.Cu) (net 15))
 (segment (start 78.800001 100) (end 82.5 103.699999) (width 0.5) (layer F.Cu) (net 15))
 (segment (start 82.5 103.75) (end 92.5 103.75) (width 0.5) (layer F.Cu) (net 15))
 (segment (start 92.5 103.75) (end 100 103.75) (width 0.5) (layer F.Cu) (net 15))
 (segment (start 78.800001 87.5) (end 82.5 91.199999) (width 0.5) (layer F.Cu) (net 13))
 (segment (start 77.5 87.5) (end 78.800001 87.5) (width 0.5) (layer F.Cu) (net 13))
 (segment (start 92.5 91.25) (end 98.75 91.25) (width 0.5) (layer F.Cu) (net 13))
 (segment (start 98.75 91.25) (end 100 91.25) (width 0.5) (layer F.Cu) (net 13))
 (segment (start 92.5 91.25) (end 82.5 91.25) (width 0.5) (layer F.Cu) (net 13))
 (segment (start 121.45 122.5) (end 121.45 127.5) (width 0.5) (layer F.Cu) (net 12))
 (segment (start 121.45 110) (end 121.45 115) (width 0.5) (layer F.Cu) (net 11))
 (segment (start 121.45 97.5) (end 121.45 102.5) (width 0.5) (layer F.Cu) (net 10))
 (segment (start 121.45 85) (end 121.45 90) (width 0.5) (layer F.Cu) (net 9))
 (segment (start 60 125) (end 64.8 125) (width 0.5) (layer F.Cu) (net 20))
 (segment (start 60 112.5) (end 65 112.5) (width 0.5) (layer F.Cu) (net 19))
 (segment (start 60 100) (end 64.8 100) (width 0.5) (layer F.Cu) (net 18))
 (segment (start 60 87.5) (end 64.8 87.5) (width 0.5) (layer F.Cu) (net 17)))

